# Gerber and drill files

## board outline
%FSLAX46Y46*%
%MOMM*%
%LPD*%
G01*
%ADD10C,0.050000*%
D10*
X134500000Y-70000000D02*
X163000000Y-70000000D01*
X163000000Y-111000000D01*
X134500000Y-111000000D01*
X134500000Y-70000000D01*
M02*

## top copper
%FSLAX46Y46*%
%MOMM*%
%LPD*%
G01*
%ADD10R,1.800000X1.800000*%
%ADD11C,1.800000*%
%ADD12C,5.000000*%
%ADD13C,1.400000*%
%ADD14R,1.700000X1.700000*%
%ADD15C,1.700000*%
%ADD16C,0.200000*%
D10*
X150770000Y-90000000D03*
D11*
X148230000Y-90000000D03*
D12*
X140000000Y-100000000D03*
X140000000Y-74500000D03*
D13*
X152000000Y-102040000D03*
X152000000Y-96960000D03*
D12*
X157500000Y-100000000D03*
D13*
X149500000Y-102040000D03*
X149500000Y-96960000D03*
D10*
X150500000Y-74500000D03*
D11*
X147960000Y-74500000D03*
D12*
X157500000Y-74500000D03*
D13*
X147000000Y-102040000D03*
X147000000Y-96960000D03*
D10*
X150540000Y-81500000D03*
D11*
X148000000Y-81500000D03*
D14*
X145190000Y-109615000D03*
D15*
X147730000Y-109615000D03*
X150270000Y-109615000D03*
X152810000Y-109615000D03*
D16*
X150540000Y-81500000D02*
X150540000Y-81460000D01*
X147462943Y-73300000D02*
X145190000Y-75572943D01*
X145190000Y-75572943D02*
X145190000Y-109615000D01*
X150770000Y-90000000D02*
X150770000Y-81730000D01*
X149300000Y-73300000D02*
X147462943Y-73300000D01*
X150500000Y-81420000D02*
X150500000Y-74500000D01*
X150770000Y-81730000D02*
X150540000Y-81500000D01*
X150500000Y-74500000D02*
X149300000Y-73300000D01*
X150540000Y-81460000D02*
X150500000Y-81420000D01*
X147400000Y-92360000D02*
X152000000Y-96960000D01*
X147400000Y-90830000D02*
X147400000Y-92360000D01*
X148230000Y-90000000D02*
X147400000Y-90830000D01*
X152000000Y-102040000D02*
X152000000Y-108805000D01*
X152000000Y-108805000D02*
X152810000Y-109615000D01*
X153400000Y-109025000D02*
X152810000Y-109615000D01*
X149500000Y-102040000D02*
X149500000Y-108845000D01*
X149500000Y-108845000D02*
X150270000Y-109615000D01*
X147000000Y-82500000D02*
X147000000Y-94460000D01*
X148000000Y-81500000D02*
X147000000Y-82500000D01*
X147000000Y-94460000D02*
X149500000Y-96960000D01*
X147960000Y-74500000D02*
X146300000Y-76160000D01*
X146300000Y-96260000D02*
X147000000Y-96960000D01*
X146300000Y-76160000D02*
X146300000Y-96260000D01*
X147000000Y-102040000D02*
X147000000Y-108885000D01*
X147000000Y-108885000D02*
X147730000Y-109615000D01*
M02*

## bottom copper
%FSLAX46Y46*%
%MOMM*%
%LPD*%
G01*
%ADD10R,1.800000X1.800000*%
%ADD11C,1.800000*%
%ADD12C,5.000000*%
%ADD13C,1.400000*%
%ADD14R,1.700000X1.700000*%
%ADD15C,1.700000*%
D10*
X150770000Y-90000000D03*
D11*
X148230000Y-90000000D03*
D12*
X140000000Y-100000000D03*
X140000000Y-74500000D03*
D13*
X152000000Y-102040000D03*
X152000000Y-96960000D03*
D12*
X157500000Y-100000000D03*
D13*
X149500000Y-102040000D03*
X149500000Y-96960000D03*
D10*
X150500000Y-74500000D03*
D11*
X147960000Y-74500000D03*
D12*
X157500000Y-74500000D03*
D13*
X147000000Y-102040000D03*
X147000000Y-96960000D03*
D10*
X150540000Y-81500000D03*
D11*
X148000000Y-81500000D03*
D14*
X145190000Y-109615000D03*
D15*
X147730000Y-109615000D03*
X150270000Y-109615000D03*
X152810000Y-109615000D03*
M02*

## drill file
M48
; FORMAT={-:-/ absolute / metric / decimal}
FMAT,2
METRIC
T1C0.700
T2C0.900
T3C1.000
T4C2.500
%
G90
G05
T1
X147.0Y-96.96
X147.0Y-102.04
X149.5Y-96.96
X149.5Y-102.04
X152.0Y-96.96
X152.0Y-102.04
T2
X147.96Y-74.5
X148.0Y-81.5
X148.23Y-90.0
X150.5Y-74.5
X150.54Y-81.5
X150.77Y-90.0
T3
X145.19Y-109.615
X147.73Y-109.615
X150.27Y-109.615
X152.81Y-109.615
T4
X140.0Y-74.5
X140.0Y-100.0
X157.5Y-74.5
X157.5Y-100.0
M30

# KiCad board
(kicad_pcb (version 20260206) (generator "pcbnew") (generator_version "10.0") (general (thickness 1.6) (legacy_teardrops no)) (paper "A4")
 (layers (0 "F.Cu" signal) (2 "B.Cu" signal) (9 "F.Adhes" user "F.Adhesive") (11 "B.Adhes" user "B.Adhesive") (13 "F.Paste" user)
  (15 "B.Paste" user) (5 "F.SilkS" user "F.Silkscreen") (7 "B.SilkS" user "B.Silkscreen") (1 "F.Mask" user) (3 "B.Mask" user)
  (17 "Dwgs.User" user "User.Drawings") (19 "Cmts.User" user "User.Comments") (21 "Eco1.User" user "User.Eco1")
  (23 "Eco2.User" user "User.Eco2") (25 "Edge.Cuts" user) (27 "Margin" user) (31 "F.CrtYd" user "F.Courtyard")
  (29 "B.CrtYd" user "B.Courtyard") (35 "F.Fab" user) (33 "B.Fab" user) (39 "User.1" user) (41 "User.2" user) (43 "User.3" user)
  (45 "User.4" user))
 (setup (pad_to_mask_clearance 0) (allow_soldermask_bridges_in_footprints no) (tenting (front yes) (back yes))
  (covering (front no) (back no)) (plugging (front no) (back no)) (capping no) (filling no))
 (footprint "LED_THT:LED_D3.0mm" (layer "F.Cu") (at 150.77 90 180)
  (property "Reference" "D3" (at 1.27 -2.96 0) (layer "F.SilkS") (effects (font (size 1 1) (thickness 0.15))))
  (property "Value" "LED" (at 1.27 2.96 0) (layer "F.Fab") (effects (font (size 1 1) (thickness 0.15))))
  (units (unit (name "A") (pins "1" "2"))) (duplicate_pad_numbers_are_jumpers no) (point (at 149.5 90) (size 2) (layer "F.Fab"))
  (pad "1" thru_hole rect (at 0 0 180) (size 1.8 1.8) (drill 0.9) (layers "*.Cu" "*.Mask") (remove_unused_layers no) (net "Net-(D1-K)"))
  (pad "2" thru_hole circle (at 2.54 0 180) (size 1.8 1.8) (drill 0.9) (layers "*.Cu" "*.Mask") (remove_unused_layers no) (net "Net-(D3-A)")))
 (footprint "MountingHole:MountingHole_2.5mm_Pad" (layer "F.Cu") (at 140 100)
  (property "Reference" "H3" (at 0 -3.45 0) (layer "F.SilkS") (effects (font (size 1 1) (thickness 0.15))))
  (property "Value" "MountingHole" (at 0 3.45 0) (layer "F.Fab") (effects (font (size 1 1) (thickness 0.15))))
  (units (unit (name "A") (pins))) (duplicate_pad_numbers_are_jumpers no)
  (pad "1" thru_hole circle (at 0 0) (size 5 5) (drill 2.5) (layers "*.Cu" "*.Mask") (remove_unused_layers no) (zone_connect 2)))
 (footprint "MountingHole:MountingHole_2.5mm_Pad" (layer "F.Cu") (at 140 74.5)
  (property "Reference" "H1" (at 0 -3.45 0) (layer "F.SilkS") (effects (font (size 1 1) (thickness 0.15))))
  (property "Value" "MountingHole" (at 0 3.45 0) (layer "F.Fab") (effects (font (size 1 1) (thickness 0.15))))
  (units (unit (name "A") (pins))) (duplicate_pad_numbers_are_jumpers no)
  (pad "1" thru_hole circle (at 0 0) (size 5 5) (drill 2.5) (layers "*.Cu" "*.Mask") (remove_unused_layers no) (zone_connect 2)))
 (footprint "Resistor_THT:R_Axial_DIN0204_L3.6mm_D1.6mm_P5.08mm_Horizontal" (layer "F.Cu") (at 152 102.04 90)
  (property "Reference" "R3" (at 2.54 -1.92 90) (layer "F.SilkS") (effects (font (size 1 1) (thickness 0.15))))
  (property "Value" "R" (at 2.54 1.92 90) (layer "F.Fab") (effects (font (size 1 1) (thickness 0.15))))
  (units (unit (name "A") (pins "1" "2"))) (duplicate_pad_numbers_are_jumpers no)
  (pad "1" thru_hole circle (at 0 0 90) (size 1.4 1.4) (drill 0.7) (layers "*.Cu" "*.Mask") (remove_unused_layers no) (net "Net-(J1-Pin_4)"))
  (pad "2" thru_hole circle (at 5.08 0 90) (size 1.4 1.4) (drill 0.7) (layers "*.Cu" "*.Mask") (remove_unused_layers no) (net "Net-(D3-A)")))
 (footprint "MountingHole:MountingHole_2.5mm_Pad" (layer "F.Cu") (at 157.5 100)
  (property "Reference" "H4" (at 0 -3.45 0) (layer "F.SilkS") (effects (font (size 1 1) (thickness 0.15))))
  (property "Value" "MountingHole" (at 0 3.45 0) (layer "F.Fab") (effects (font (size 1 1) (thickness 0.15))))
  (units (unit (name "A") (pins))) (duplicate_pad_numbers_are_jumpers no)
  (pad "1" thru_hole circle (at 0 0) (size 5 5) (drill 2.5) (layers "*.Cu" "*.Mask") (remove_unused_layers no) (zone_connect 2)))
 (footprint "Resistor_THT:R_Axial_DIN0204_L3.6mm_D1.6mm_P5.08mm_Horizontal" (layer "F.Cu") (at 149.5 102.04 90)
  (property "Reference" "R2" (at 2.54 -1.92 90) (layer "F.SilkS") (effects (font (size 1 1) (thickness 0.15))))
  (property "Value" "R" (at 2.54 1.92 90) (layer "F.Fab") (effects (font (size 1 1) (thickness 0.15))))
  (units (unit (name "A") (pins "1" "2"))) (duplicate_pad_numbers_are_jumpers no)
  (pad "1" thru_hole circle (at 0 0 90) (size 1.4 1.4) (drill 0.7) (layers "*.Cu" "*.Mask") (remove_unused_layers no) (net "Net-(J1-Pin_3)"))
  (pad "2" thru_hole circle (at 5.08 0 90) (size 1.4 1.4) (drill 0.7) (layers "*.Cu" "*.Mask") (remove_unused_layers no) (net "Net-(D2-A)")))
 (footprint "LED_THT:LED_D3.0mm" (layer "F.Cu") (at 150.5 74.5 180)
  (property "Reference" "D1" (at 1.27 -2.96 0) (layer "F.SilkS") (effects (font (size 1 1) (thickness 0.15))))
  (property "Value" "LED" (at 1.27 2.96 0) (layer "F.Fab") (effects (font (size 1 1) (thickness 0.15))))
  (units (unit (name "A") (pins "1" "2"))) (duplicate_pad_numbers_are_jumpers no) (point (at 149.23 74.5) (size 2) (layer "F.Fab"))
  (pad "1" thru_hole rect (at 0 0 180) (size 1.8 1.8) (drill 0.9) (layers "*.Cu" "*.Mask") (remove_unused_layers no) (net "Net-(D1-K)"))
  (pad "2" thru_hole circle (at 2.54 0 180) (size 1.8 1.8) (drill 0.9) (layers "*.Cu" "*.Mask") (remove_unused_layers no) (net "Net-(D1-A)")))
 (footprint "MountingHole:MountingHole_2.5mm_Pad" (layer "F.Cu") (at 157.5 74.5)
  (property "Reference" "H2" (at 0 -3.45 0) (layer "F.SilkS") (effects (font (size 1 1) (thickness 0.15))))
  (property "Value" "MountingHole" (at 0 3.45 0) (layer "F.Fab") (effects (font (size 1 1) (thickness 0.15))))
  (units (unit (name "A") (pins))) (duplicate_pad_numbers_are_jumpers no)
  (pad "1" thru_hole circle (at 0 0) (size 5 5) (drill 2.5) (layers "*.Cu" "*.Mask") (remove_unused_layers no) (zone_connect 2)))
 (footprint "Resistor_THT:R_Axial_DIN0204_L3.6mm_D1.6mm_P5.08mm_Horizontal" (layer "F.Cu") (at 147 102.04 90)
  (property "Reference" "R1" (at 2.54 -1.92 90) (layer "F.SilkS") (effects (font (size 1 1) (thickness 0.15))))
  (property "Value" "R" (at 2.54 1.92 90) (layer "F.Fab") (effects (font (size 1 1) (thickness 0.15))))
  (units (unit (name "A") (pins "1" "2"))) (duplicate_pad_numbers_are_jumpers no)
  (pad "1" thru_hole circle (at 0 0 90) (size 1.4 1.4) (drill 0.7) (layers "*.Cu" "*.Mask") (remove_unused_layers no) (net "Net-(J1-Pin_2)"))
  (pad "2" thru_hole circle (at 5.08 0 90) (size 1.4 1.4) (drill 0.7) (layers "*.Cu" "*.Mask") (remove_unused_layers no) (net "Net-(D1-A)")))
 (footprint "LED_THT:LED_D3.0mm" (layer "F.Cu") (at 150.54 81.5 180)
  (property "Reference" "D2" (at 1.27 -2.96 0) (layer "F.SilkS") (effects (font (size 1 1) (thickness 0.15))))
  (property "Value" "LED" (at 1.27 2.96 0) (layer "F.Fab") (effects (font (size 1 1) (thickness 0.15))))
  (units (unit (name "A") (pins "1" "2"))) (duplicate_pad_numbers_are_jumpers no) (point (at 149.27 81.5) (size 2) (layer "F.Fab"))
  (pad "1" thru_hole rect (at 0 0 180) (size 1.8 1.8) (drill 0.9) (layers "*.Cu" "*.Mask") (remove_unused_layers no) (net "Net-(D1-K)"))
  (pad "2" thru_hole circle (at 2.54 0 180) (size 1.8 1.8) (drill 0.9) (layers "*.Cu" "*.Mask") (remove_unused_layers no) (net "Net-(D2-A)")))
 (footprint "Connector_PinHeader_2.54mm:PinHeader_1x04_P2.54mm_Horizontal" (layer "B.Cu") (at 145.19 109.615 -90)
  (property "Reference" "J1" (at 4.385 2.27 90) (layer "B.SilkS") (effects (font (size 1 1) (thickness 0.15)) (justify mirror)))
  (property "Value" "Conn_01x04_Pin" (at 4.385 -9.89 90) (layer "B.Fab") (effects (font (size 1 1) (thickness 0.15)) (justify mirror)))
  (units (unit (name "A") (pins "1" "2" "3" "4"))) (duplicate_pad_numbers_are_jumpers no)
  (pad "1" thru_hole rect (at 0 0 270) (size 1.7 1.7) (drill 1) (layers "*.Cu" "*.Mask") (remove_unused_layers no) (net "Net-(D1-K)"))
  (pad "2" thru_hole circle (at 0 -2.54 270) (size 1.7 1.7) (drill 1) (layers "*.Cu" "*.Mask") (remove_unused_layers no)
   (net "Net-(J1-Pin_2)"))
  (pad "3" thru_hole circle (at 0 -5.08 270) (size 1.7 1.7) (drill 1) (layers "*.Cu" "*.Mask") (remove_unused_layers no)
   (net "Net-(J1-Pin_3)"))
  (pad "4" thru_hole circle (at 0 -7.62 270) (size 1.7 1.7) (drill 1) (layers "*.Cu" "*.Mask") (remove_unused_layers no)
   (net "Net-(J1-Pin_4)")))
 (gr_rect (start 134.5 70) (end 163 111) (stroke (width 0.05) (type default)) (fill no) (layer "Edge.Cuts"))
 (segment (start 150.54 81.5) (end 150.54 81.46) (width 0.2) (layer "F.Cu") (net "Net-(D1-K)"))
 (segment (start 147.462943 73.3) (end 145.19 75.572943) (width 0.2) (layer "F.Cu") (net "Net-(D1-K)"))
 (segment (start 145.19 75.572943) (end 145.19 109.615) (width 0.2) (layer "F.Cu") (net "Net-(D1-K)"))
 (segment (start 150.77 90) (end 150.77 81.73) (width 0.2) (layer "F.Cu") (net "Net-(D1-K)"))
 (segment (start 149.3 73.3) (end 147.462943 73.3) (width 0.2) (layer "F.Cu") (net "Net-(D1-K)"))
 (segment (start 150.5 81.42) (end 150.5 74.5) (width 0.2) (layer "F.Cu") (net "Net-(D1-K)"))
 (segment (start 150.77 81.73) (end 150.54 81.5) (width 0.2) (layer "F.Cu") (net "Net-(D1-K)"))
 (segment (start 150.5 74.5) (end 149.3 73.3) (width 0.2) (layer "F.Cu") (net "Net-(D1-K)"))
 (segment (start 150.54 81.46) (end 150.5 81.42) (width 0.2) (layer "F.Cu") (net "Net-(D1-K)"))
 (segment (start 147.4 92.36) (end 152 96.96) (width 0.2) (layer "F.Cu") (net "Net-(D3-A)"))
 (segment (start 147.4 90.83) (end 147.4 92.36) (width 0.2) (layer "F.Cu") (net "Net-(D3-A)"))
 (segment (start 148.23 90) (end 147.4 90.83) (width 0.2) (layer "F.Cu") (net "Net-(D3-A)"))
 (segment (start 152 102.04) (end 152 108.805) (width 0.2) (layer "F.Cu") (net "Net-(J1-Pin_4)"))
 (segment (start 152 108.805) (end 152.81 109.615) (width 0.2) (layer "F.Cu") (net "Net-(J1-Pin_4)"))
 (segment (start 153.4 109.025) (end 152.81 109.615) (width 0.2) (layer "F.Cu") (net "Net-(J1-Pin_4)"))
 (segment (start 149.5 102.04) (end 149.5 108.845) (width 0.2) (layer "F.Cu") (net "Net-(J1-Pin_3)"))
 (segment (start 149.5 108.845) (end 150.27 109.615) (width 0.2) (layer "F.Cu") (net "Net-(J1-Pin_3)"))
 (segment (start 147 82.5) (end 147 94.46) (width 0.2) (layer "F.Cu") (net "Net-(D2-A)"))
 (segment (start 148 81.5) (end 147 82.5) (width 0.2) (layer "F.Cu") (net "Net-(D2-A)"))
 (segment (start 147 94.46) (end 149.5 96.96) (width 0.2) (layer "F.Cu") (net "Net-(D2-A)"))
 (segment (start 147.96 74.5) (end 146.3 76.16) (width 0.2) (layer "F.Cu") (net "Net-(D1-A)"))
 (segment (start 146.3 96.26) (end 147 96.96) (width 0.2) (layer "F.Cu") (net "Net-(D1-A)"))
 (segment (start 146.3 76.16) (end 146.3 96.26) (width 0.2) (layer "F.Cu") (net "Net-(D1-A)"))
 (segment (start 147 102.04) (end 147 108.885) (width 0.2) (layer "F.Cu") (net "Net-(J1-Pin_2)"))
 (segment (start 147 108.885) (end 147.73 109.615) (width 0.2) (layer "F.Cu") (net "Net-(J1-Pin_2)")))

